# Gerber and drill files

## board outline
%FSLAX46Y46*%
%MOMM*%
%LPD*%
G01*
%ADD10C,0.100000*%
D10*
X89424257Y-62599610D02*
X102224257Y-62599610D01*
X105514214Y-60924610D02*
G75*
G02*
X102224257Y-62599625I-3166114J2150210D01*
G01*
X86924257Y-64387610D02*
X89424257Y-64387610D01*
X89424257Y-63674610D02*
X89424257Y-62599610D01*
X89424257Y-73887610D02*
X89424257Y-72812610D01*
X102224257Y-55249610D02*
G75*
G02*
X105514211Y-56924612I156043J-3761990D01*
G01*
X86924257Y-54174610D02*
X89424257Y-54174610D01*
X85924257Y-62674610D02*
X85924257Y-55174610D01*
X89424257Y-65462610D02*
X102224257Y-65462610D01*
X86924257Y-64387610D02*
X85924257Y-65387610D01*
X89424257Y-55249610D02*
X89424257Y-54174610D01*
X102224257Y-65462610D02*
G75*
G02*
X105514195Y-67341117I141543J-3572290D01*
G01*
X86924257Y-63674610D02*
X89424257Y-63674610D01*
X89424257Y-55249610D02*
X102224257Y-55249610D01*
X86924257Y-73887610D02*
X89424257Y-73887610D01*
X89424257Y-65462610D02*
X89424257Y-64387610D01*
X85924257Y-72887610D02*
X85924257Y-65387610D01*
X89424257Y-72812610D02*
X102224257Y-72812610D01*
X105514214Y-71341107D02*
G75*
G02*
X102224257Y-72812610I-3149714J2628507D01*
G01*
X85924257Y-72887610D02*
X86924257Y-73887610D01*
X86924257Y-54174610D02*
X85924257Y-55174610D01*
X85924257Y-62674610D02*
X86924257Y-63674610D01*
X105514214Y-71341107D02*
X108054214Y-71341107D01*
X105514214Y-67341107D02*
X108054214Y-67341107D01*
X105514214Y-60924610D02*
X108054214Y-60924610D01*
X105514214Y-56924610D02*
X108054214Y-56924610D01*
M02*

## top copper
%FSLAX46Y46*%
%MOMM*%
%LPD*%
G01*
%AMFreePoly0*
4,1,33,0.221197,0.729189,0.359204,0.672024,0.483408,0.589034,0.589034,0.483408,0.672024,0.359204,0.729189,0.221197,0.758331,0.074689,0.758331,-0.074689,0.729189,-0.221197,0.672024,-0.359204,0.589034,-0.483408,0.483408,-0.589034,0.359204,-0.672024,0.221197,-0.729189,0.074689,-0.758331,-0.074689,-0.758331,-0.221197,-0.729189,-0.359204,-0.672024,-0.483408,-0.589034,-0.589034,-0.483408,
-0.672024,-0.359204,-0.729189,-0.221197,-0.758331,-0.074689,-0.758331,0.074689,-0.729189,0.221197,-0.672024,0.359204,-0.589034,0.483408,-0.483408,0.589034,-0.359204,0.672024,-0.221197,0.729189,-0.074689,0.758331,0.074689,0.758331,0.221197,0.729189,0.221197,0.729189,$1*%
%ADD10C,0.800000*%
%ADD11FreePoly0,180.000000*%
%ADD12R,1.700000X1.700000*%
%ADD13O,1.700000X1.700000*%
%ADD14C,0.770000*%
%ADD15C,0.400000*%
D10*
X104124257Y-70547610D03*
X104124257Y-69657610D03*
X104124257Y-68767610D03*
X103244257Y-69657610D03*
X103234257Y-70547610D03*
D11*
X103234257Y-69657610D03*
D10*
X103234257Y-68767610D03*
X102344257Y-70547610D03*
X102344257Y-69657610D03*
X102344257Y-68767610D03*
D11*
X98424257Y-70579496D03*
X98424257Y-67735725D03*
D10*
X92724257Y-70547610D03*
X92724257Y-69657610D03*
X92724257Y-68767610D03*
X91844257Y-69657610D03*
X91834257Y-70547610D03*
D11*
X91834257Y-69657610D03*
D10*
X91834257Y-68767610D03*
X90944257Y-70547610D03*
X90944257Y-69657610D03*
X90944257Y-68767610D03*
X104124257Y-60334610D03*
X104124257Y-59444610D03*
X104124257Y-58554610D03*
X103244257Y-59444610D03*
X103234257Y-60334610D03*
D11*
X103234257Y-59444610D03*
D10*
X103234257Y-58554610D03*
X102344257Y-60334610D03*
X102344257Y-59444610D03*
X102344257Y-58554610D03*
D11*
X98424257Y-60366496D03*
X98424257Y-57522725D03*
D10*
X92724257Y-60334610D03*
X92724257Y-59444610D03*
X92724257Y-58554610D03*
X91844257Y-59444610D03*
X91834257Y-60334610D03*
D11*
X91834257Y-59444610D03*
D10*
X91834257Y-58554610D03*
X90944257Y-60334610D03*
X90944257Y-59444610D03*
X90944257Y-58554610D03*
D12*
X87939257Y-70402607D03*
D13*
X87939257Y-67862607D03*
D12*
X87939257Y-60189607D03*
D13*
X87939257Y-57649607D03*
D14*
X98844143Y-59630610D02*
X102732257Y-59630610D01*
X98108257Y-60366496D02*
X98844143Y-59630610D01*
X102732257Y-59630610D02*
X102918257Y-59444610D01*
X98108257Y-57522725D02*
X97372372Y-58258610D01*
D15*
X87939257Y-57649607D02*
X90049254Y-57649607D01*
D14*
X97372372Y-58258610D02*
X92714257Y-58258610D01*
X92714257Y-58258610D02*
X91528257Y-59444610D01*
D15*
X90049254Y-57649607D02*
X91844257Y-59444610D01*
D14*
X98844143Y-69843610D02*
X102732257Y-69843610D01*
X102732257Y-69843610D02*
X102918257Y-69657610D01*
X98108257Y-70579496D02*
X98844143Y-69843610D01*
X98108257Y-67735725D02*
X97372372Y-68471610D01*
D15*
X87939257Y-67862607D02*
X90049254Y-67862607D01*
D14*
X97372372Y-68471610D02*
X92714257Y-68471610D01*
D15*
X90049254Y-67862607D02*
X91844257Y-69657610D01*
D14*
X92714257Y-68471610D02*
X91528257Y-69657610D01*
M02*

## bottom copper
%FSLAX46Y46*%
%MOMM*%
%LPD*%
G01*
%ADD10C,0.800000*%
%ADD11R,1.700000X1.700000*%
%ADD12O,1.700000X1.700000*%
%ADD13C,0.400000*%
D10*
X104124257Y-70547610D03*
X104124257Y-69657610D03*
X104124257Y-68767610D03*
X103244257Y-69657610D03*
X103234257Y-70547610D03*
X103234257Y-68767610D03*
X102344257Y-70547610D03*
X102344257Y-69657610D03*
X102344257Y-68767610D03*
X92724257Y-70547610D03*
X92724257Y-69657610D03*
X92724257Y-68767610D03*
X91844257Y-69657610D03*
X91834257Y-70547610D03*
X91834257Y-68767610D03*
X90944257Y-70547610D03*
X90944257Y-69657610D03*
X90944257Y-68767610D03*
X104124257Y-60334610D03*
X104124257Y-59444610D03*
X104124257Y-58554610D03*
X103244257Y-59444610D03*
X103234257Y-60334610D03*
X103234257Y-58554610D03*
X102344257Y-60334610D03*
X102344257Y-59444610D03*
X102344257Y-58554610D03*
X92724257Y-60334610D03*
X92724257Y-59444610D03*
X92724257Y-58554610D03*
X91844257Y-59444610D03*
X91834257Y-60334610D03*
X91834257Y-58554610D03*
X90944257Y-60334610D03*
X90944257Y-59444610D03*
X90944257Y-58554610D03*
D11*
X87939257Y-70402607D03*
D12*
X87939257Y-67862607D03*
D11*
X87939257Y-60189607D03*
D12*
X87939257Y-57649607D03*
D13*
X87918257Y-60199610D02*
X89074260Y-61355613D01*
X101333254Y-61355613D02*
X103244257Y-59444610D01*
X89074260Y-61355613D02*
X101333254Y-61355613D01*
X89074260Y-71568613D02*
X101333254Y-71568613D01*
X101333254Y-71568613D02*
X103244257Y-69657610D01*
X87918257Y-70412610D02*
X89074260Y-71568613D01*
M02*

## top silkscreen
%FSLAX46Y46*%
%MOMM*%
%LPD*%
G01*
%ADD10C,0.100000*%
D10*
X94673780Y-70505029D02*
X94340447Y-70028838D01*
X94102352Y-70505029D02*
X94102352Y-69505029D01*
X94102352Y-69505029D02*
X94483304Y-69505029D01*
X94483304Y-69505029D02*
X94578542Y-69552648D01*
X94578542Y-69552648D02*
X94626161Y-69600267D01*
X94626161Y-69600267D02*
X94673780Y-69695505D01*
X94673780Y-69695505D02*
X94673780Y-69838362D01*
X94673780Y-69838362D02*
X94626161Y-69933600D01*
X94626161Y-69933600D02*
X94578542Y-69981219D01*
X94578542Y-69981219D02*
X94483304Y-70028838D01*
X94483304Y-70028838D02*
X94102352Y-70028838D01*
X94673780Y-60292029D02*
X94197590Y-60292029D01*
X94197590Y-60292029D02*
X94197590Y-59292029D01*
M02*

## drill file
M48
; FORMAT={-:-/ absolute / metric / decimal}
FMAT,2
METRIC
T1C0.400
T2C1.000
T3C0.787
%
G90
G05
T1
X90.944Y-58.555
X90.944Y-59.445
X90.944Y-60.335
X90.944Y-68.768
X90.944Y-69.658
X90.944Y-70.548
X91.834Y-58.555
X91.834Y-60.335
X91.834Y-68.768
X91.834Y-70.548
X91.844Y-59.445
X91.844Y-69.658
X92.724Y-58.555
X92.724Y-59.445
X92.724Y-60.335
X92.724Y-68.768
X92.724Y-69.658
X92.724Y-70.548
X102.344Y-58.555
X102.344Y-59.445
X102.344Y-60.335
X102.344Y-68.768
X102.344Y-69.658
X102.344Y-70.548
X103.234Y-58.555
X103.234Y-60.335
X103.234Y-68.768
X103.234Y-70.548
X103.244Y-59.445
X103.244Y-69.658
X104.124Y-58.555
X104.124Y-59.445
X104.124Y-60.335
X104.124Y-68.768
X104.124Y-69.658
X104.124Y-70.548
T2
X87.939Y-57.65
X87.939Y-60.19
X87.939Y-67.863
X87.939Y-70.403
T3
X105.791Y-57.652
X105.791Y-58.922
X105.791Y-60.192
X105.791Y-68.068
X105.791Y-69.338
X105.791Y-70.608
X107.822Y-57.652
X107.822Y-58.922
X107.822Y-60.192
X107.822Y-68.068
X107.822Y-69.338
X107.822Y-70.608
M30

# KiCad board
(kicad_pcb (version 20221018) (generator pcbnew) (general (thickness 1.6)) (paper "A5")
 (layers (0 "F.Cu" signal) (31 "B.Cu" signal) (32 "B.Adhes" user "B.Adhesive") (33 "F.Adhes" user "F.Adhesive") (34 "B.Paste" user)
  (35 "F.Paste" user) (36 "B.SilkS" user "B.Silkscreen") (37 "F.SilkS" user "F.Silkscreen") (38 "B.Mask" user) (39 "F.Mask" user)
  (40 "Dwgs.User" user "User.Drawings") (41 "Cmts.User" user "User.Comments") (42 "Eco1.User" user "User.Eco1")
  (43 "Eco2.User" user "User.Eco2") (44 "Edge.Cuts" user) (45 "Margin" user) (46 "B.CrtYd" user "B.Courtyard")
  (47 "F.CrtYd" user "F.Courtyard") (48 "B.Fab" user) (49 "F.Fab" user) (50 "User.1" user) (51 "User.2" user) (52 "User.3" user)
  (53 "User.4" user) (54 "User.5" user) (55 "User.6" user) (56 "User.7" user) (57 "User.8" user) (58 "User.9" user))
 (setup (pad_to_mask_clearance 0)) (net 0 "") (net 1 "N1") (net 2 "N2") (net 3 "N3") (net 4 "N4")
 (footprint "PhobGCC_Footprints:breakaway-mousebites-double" (layer "F.Cu") (at 108.052107 69.108107 90)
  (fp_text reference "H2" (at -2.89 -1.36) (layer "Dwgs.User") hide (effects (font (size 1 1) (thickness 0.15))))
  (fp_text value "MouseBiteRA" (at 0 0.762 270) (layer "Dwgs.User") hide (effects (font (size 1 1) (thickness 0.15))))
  (fp_line (start -2.233 -2.537893) (end -2.233 0.002107) (stroke (width 0.1) (type solid)) (layer "Edge.Cuts"))
  (fp_line (start 1.767 -2.537893) (end 1.767 0.002107) (stroke (width 0.1) (type solid)) (layer "Edge.Cuts"))
  (pad "" np_thru_hole circle (at -1.5 -2.26085 270) (size 0.7874 0.7874) (drill 0.7874) (layers "*.Cu" "*.Mask"))
  (pad "" np_thru_hole circle (at -1.5 -0.23 90) (size 0.7874 0.7874) (drill 0.7874) (layers "*.Cu" "*.Mask"))
  (pad "" np_thru_hole circle (at -0.23 -2.26085 270) (size 0.7874 0.7874) (drill 0.7874) (layers "*.Cu" "*.Mask"))
  (pad "" np_thru_hole circle (at -0.23 -0.23 90) (size 0.7874 0.7874) (drill 0.7874) (layers "*.Cu" "*.Mask"))
  (pad "" np_thru_hole circle (at 1.04 -2.26085 270) (size 0.7874 0.7874) (drill 0.7874) (layers "*.Cu" "*.Mask"))
  (pad "" np_thru_hole circle (at 1.04 -0.23 90) (size 0.7874 0.7874) (drill 0.7874) (layers "*.Cu" "*.Mask")))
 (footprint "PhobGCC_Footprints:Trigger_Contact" (layer "F.Cu") (at 98.424257 69.15761 180)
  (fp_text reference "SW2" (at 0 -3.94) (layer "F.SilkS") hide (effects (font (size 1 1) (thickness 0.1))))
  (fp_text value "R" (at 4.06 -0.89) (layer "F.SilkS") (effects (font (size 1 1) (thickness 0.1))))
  (pad "1" thru_hole circle (at -5.7 -1.39 180) (size 0.8 0.8) (drill 0.4) (layers "*.Cu" "*.Mask") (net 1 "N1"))
  (pad "1" thru_hole circle (at -5.7 -0.5 180) (size 0.8 0.8) (drill 0.4) (layers "*.Cu" "*.Mask") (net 1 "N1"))
  (pad "1" thru_hole circle (at -5.7 0.39 180) (size 0.8 0.8) (drill 0.4) (layers "*.Cu" "*.Mask") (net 1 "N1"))
  (pad "1" thru_hole circle (at -4.82 -0.5 180) (size 0.8 0.8) (drill 0.4) (layers "*.Cu" "*.Mask") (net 1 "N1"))
  (pad "1" thru_hole circle (at -4.81 -1.39 180) (size 0.8 0.8) (drill 0.4) (layers "*.Cu" "*.Mask") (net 1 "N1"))
  (pad "1" smd custom (at -4.81 -0.5 180) (size 1.524 1.524) (layers "F.Cu" "F.Paste" "F.Mask") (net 1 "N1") (thermal_bridge_angle 45)
   (options (clearance outline) (anchor circle)) (primitives))
  (pad "1" thru_hole circle (at -4.81 0.39 180) (size 0.8 0.8) (drill 0.4) (layers "*.Cu" "*.Mask") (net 1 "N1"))
  (pad "1" thru_hole circle (at -3.92 -1.39 180) (size 0.8 0.8) (drill 0.4) (layers "*.Cu" "*.Mask") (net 1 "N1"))
  (pad "1" thru_hole circle (at -3.92 -0.5 180) (size 0.8 0.8) (drill 0.4) (layers "*.Cu" "*.Mask") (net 1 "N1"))
  (pad "1" thru_hole circle (at -3.92 0.39 180) (size 0.8 0.8) (drill 0.4) (layers "*.Cu" "*.Mask") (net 1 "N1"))
  (pad "1" smd custom (at 0 -1.421886 180) (size 1.524 1.524) (layers "F.Cu" "F.Paste" "F.Mask") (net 1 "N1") (thermal_bridge_angle 45)
   (options (clearance outline) (anchor circle)) (primitives))
  (pad "2" smd custom (at 0 1.421885 180) (size 1.524 1.524) (layers "F.Cu" "F.Paste" "F.Mask") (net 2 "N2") (thermal_bridge_angle 45)
   (options (clearance outline) (anchor circle)) (primitives))
  (pad "2" thru_hole circle (at 5.7 -1.39 180) (size 0.8 0.8) (drill 0.4) (layers "*.Cu" "*.Mask") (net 2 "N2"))
  (pad "2" thru_hole circle (at 5.7 -0.5 180) (size 0.8 0.8) (drill 0.4) (layers "*.Cu" "*.Mask") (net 2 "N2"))
  (pad "2" thru_hole circle (at 5.7 0.39 180) (size 0.8 0.8) (drill 0.4) (layers "*.Cu" "*.Mask") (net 2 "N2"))
  (pad "2" thru_hole circle (at 6.58 -0.5 180) (size 0.8 0.8) (drill 0.4) (layers "*.Cu" "*.Mask") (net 2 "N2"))
  (pad "2" thru_hole circle (at 6.59 -1.39 180) (size 0.8 0.8) (drill 0.4) (layers "*.Cu" "*.Mask") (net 2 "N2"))
  (pad "2" smd custom (at 6.59 -0.5 180) (size 1.524 1.524) (layers "F.Cu" "F.Paste" "F.Mask") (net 2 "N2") (thermal_bridge_angle 45)
   (options (clearance outline) (anchor circle)) (primitives))
  (pad "2" thru_hole circle (at 6.59 0.39 180) (size 0.8 0.8) (drill 0.4) (layers "*.Cu" "*.Mask") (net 2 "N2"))
  (pad "2" thru_hole circle (at 7.48 -1.39 180) (size 0.8 0.8) (drill 0.4) (layers "*.Cu" "*.Mask") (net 2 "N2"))
  (pad "2" thru_hole circle (at 7.48 -0.5 180) (size 0.8 0.8) (drill 0.4) (layers "*.Cu" "*.Mask") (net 2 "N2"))
  (pad "2" thru_hole circle (at 7.48 0.39 180) (size 0.8 0.8) (drill 0.4) (layers "*.Cu" "*.Mask") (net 2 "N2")))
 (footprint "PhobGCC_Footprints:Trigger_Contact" (layer "F.Cu") (at 98.424257 58.94461 180)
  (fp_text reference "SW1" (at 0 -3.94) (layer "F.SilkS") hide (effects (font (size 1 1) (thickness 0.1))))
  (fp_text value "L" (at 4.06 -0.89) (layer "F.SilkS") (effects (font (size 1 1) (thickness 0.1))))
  (pad "1" thru_hole circle (at -5.7 -1.39 180) (size 0.8 0.8) (drill 0.4) (layers "*.Cu" "*.Mask") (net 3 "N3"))
  (pad "1" thru_hole circle (at -5.7 -0.5 180) (size 0.8 0.8) (drill 0.4) (layers "*.Cu" "*.Mask") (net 3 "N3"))
  (pad "1" thru_hole circle (at -5.7 0.39 180) (size 0.8 0.8) (drill 0.4) (layers "*.Cu" "*.Mask") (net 3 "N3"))
  (pad "1" thru_hole circle (at -4.82 -0.5 180) (size 0.8 0.8) (drill 0.4) (layers "*.Cu" "*.Mask") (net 3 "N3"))
  (pad "1" thru_hole circle (at -4.81 -1.39 180) (size 0.8 0.8) (drill 0.4) (layers "*.Cu" "*.Mask") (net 3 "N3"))
  (pad "1" smd custom (at -4.81 -0.5 180) (size 1.524 1.524) (layers "F.Cu" "F.Paste" "F.Mask") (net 3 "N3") (thermal_bridge_angle 45)
   (options (clearance outline) (anchor circle)) (primitives))
  (pad "1" thru_hole circle (at -4.81 0.39 180) (size 0.8 0.8) (drill 0.4) (layers "*.Cu" "*.Mask") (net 3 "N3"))
  (pad "1" thru_hole circle (at -3.92 -1.39 180) (size 0.8 0.8) (drill 0.4) (layers "*.Cu" "*.Mask") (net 3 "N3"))
  (pad "1" thru_hole circle (at -3.92 -0.5 180) (size 0.8 0.8) (drill 0.4) (layers "*.Cu" "*.Mask") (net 3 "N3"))
  (pad "1" thru_hole circle (at -3.92 0.39 180) (size 0.8 0.8) (drill 0.4) (layers "*.Cu" "*.Mask") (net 3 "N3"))
  (pad "1" smd custom (at 0 -1.421886 180) (size 1.524 1.524) (layers "F.Cu" "F.Paste" "F.Mask") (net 3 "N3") (thermal_bridge_angle 45)
   (options (clearance outline) (anchor circle)) (primitives))
  (pad "2" smd custom (at 0 1.421885 180) (size 1.524 1.524) (layers "F.Cu" "F.Paste" "F.Mask") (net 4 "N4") (thermal_bridge_angle 45)
   (options (clearance outline) (anchor circle)) (primitives))
  (pad "2" thru_hole circle (at 5.7 -1.39 180) (size 0.8 0.8) (drill 0.4) (layers "*.Cu" "*.Mask") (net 4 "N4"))
  (pad "2" thru_hole circle (at 5.7 -0.5 180) (size 0.8 0.8) (drill 0.4) (layers "*.Cu" "*.Mask") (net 4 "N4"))
  (pad "2" thru_hole circle (at 5.7 0.39 180) (size 0.8 0.8) (drill 0.4) (layers "*.Cu" "*.Mask") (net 4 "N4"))
  (pad "2" thru_hole circle (at 6.58 -0.5 180) (size 0.8 0.8) (drill 0.4) (layers "*.Cu" "*.Mask") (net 4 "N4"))
  (pad "2" thru_hole circle (at 6.59 -1.39 180) (size 0.8 0.8) (drill 0.4) (layers "*.Cu" "*.Mask") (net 4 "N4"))
  (pad "2" smd custom (at 6.59 -0.5 180) (size 1.524 1.524) (layers "F.Cu" "F.Paste" "F.Mask") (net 4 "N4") (thermal_bridge_angle 45)
   (options (clearance outline) (anchor circle)) (primitives))
  (pad "2" thru_hole circle (at 6.59 0.39 180) (size 0.8 0.8) (drill 0.4) (layers "*.Cu" "*.Mask") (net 4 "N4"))
  (pad "2" thru_hole circle (at 7.48 -1.39 180) (size 0.8 0.8) (drill 0.4) (layers "*.Cu" "*.Mask") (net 4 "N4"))
  (pad "2" thru_hole circle (at 7.48 -0.5 180) (size 0.8 0.8) (drill 0.4) (layers "*.Cu" "*.Mask") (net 4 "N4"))
  (pad "2" thru_hole circle (at 7.48 0.39 180) (size 0.8 0.8) (drill 0.4) (layers "*.Cu" "*.Mask") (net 4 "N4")))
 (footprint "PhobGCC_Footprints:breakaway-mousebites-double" (layer "F.Cu") (at 108.052107 58.69161 90)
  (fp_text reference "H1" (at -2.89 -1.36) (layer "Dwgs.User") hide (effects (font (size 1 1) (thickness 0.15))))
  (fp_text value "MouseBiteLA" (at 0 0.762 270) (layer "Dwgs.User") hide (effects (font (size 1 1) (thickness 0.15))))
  (fp_line (start -2.233 -2.537893) (end -2.233 0.002107) (stroke (width 0.1) (type solid)) (layer "Edge.Cuts"))
  (fp_line (start 1.767 -2.537893) (end 1.767 0.002107) (stroke (width 0.1) (type solid)) (layer "Edge.Cuts"))
  (pad "" np_thru_hole circle (at -1.5 -2.26085 270) (size 0.7874 0.7874) (drill 0.7874) (layers "*.Cu" "*.Mask"))
  (pad "" np_thru_hole circle (at -1.5 -0.23 90) (size 0.7874 0.7874) (drill 0.7874) (layers "*.Cu" "*.Mask"))
  (pad "" np_thru_hole circle (at -0.23 -2.26085 270) (size 0.7874 0.7874) (drill 0.7874) (layers "*.Cu" "*.Mask"))
  (pad "" np_thru_hole circle (at -0.23 -0.23 90) (size 0.7874 0.7874) (drill 0.7874) (layers "*.Cu" "*.Mask"))
  (pad "" np_thru_hole circle (at 1.04 -2.26085 270) (size 0.7874 0.7874) (drill 0.7874) (layers "*.Cu" "*.Mask"))
  (pad "" np_thru_hole circle (at 1.04 -0.23 90) (size 0.7874 0.7874) (drill 0.7874) (layers "*.Cu" "*.Mask")))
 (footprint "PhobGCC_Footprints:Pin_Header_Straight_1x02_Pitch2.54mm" (layer "B.Cu") (at 87.939257 70.402607)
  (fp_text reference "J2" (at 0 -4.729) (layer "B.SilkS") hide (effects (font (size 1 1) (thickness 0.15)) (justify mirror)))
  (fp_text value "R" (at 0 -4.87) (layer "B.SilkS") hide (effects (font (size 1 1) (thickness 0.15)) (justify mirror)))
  (pad "1" thru_hole rect (at 0 0) (size 1.7 1.7) (drill 1) (layers "*.Cu" "*.Mask") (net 1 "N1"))
  (pad "2" thru_hole oval (at 0 -2.54) (size 1.7 1.7) (drill 1) (layers "*.Cu" "*.Mask") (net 2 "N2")))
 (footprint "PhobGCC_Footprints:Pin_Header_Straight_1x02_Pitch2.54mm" (layer "B.Cu") (at 87.939257 60.189607)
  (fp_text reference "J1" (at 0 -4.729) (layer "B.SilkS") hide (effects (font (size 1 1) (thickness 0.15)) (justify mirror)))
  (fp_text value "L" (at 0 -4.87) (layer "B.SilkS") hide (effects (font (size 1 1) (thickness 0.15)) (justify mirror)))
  (pad "1" thru_hole rect (at 0 0) (size 1.7 1.7) (drill 1) (layers "*.Cu" "*.Mask") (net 3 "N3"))
  (pad "2" thru_hole oval (at 0 -2.54) (size 1.7 1.7) (drill 1) (layers "*.Cu" "*.Mask") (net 4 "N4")))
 (gr_line (start 89.424257 62.59961) (end 102.224257 62.59961) (stroke (width 0.1) (type solid)) (layer "Edge.Cuts"))
 (gr_arc (start 105.514214 60.92461) (mid 104.084555 62.18503) (end 102.224257 62.59961) (stroke (width 0.1) (type solid))
  (layer "Edge.Cuts"))
 (gr_line (start 86.924257 64.38761) (end 89.424257 64.38761) (stroke (width 0.1) (type solid)) (layer "Edge.Cuts"))
 (gr_line (start 89.424257 63.67461) (end 89.424257 62.59961) (stroke (width 0.1) (type solid)) (layer "Edge.Cuts"))
 (gr_line (start 89.424257 73.88761) (end 89.424257 72.81261) (stroke (width 0.1) (type solid)) (layer "Edge.Cuts"))
 (gr_arc (start 102.224257 55.24961) (mid 104.088615 55.656215) (end 105.514214 56.92461) (stroke (width 0.1) (type solid))
  (layer "Edge.Cuts"))
 (gr_line (start 86.924257 54.17461) (end 89.424257 54.17461) (stroke (width 0.1) (type solid)) (layer "Edge.Cuts"))
 (gr_line (start 85.924257 62.67461) (end 85.924257 55.17461) (stroke (width 0.1) (type solid)) (layer "Edge.Cuts"))
 (gr_line (start 89.424257 65.46261) (end 102.224257 65.46261) (stroke (width 0.1) (type solid)) (layer "Edge.Cuts"))
 (gr_line (start 86.924257 64.38761) (end 85.924257 65.38761) (stroke (width 0.1) (type solid)) (layer "Edge.Cuts"))
 (gr_line (start 89.424257 55.24961) (end 89.424257 54.17461) (stroke (width 0.1) (type solid)) (layer "Edge.Cuts"))
 (gr_arc (start 102.224257 65.46261) (mid 104.138511 65.930255) (end 105.514214 67.341107) (stroke (width 0.1) (type solid))
  (layer "Edge.Cuts"))
 (gr_line (start 86.924257 63.67461) (end 89.424257 63.67461) (stroke (width 0.1) (type solid)) (layer "Edge.Cuts"))
 (gr_line (start 89.424257 55.24961) (end 102.224257 55.24961) (stroke (width 0.1) (type solid)) (layer "Edge.Cuts"))
 (gr_line (start 86.924257 73.88761) (end 89.424257 73.88761) (stroke (width 0.1) (type solid)) (layer "Edge.Cuts"))
 (gr_line (start 89.424257 65.46261) (end 89.424257 64.38761) (stroke (width 0.1) (type solid)) (layer "Edge.Cuts"))
 (gr_line (start 85.924257 72.88761) (end 85.924257 65.38761) (stroke (width 0.1) (type solid)) (layer "Edge.Cuts"))
 (gr_line (start 89.424257 72.81261) (end 102.224257 72.81261) (stroke (width 0.1) (type solid)) (layer "Edge.Cuts"))
 (gr_arc (start 105.514214 71.341107) (mid 104.03948 72.457488) (end 102.224257 72.81261) (stroke (width 0.1) (type solid))
  (layer "Edge.Cuts"))
 (gr_line (start 85.924257 72.88761) (end 86.924257 73.88761) (stroke (width 0.1) (type solid)) (layer "Edge.Cuts"))
 (gr_line (start 86.924257 54.17461) (end 85.924257 55.17461) (stroke (width 0.1) (type solid)) (layer "Edge.Cuts"))
 (gr_line (start 85.924257 62.67461) (end 86.924257 63.67461) (stroke (width 0.1) (type solid)) (layer "Edge.Cuts"))
 (segment (start 98.844143 59.63061) (end 102.732257 59.63061) (width 0.77) (layer "F.Cu") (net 3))
 (segment (start 98.108257 60.366496) (end 98.844143 59.63061) (width 0.77) (layer "F.Cu") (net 3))
 (segment (start 102.732257 59.63061) (end 102.918257 59.44461) (width 0.77) (layer "F.Cu") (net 3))
 (segment (start 87.918257 60.19961) (end 89.07426 61.355613) (width 0.4) (layer "B.Cu") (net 3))
 (segment (start 101.333254 61.355613) (end 103.244257 59.44461) (width 0.4) (layer "B.Cu") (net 3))
 (segment (start 89.07426 61.355613) (end 101.333254 61.355613) (width 0.4) (layer "B.Cu") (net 3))
 (segment (start 98.108257 57.522725) (end 97.372372 58.25861) (width 0.77) (layer "F.Cu") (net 4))
 (segment (start 87.939257 57.649607) (end 90.049254 57.649607) (width 0.4) (layer "F.Cu") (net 4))
 (segment (start 97.372372 58.25861) (end 92.714257 58.25861) (width 0.77) (layer "F.Cu") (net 4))
 (segment (start 92.714257 58.25861) (end 91.528257 59.44461) (width 0.77) (layer "F.Cu") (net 4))
 (segment (start 90.049254 57.649607) (end 91.844257 59.44461) (width 0.4) (layer "F.Cu") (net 4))
 (segment (start 98.844143 69.84361) (end 102.732257 69.84361) (width 0.77) (layer "F.Cu") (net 1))
 (segment (start 102.732257 69.84361) (end 102.918257 69.65761) (width 0.77) (layer "F.Cu") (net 1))
 (segment (start 98.108257 70.579496) (end 98.844143 69.84361) (width 0.77) (layer "F.Cu") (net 1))
 (segment (start 89.07426 71.568613) (end 101.333254 71.568613) (width 0.4) (layer "B.Cu") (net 1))
 (segment (start 101.333254 71.568613) (end 103.244257 69.65761) (width 0.4) (layer "B.Cu") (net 1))
 (segment (start 87.918257 70.41261) (end 89.07426 71.568613) (width 0.4) (layer "B.Cu") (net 1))
 (segment (start 98.108257 67.735725) (end 97.372372 68.47161) (width 0.77) (layer "F.Cu") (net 2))
 (segment (start 87.939257 67.862607) (end 90.049254 67.862607) (width 0.4) (layer "F.Cu") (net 2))
 (segment (start 97.372372 68.47161) (end 92.714257 68.47161) (width 0.77) (layer "F.Cu") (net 2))
 (segment (start 90.049254 67.862607) (end 91.844257 69.65761) (width 0.4) (layer "F.Cu") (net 2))
 (segment (start 92.714257 68.47161) (end 91.528257 69.65761) (width 0.77) (layer "F.Cu") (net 2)))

